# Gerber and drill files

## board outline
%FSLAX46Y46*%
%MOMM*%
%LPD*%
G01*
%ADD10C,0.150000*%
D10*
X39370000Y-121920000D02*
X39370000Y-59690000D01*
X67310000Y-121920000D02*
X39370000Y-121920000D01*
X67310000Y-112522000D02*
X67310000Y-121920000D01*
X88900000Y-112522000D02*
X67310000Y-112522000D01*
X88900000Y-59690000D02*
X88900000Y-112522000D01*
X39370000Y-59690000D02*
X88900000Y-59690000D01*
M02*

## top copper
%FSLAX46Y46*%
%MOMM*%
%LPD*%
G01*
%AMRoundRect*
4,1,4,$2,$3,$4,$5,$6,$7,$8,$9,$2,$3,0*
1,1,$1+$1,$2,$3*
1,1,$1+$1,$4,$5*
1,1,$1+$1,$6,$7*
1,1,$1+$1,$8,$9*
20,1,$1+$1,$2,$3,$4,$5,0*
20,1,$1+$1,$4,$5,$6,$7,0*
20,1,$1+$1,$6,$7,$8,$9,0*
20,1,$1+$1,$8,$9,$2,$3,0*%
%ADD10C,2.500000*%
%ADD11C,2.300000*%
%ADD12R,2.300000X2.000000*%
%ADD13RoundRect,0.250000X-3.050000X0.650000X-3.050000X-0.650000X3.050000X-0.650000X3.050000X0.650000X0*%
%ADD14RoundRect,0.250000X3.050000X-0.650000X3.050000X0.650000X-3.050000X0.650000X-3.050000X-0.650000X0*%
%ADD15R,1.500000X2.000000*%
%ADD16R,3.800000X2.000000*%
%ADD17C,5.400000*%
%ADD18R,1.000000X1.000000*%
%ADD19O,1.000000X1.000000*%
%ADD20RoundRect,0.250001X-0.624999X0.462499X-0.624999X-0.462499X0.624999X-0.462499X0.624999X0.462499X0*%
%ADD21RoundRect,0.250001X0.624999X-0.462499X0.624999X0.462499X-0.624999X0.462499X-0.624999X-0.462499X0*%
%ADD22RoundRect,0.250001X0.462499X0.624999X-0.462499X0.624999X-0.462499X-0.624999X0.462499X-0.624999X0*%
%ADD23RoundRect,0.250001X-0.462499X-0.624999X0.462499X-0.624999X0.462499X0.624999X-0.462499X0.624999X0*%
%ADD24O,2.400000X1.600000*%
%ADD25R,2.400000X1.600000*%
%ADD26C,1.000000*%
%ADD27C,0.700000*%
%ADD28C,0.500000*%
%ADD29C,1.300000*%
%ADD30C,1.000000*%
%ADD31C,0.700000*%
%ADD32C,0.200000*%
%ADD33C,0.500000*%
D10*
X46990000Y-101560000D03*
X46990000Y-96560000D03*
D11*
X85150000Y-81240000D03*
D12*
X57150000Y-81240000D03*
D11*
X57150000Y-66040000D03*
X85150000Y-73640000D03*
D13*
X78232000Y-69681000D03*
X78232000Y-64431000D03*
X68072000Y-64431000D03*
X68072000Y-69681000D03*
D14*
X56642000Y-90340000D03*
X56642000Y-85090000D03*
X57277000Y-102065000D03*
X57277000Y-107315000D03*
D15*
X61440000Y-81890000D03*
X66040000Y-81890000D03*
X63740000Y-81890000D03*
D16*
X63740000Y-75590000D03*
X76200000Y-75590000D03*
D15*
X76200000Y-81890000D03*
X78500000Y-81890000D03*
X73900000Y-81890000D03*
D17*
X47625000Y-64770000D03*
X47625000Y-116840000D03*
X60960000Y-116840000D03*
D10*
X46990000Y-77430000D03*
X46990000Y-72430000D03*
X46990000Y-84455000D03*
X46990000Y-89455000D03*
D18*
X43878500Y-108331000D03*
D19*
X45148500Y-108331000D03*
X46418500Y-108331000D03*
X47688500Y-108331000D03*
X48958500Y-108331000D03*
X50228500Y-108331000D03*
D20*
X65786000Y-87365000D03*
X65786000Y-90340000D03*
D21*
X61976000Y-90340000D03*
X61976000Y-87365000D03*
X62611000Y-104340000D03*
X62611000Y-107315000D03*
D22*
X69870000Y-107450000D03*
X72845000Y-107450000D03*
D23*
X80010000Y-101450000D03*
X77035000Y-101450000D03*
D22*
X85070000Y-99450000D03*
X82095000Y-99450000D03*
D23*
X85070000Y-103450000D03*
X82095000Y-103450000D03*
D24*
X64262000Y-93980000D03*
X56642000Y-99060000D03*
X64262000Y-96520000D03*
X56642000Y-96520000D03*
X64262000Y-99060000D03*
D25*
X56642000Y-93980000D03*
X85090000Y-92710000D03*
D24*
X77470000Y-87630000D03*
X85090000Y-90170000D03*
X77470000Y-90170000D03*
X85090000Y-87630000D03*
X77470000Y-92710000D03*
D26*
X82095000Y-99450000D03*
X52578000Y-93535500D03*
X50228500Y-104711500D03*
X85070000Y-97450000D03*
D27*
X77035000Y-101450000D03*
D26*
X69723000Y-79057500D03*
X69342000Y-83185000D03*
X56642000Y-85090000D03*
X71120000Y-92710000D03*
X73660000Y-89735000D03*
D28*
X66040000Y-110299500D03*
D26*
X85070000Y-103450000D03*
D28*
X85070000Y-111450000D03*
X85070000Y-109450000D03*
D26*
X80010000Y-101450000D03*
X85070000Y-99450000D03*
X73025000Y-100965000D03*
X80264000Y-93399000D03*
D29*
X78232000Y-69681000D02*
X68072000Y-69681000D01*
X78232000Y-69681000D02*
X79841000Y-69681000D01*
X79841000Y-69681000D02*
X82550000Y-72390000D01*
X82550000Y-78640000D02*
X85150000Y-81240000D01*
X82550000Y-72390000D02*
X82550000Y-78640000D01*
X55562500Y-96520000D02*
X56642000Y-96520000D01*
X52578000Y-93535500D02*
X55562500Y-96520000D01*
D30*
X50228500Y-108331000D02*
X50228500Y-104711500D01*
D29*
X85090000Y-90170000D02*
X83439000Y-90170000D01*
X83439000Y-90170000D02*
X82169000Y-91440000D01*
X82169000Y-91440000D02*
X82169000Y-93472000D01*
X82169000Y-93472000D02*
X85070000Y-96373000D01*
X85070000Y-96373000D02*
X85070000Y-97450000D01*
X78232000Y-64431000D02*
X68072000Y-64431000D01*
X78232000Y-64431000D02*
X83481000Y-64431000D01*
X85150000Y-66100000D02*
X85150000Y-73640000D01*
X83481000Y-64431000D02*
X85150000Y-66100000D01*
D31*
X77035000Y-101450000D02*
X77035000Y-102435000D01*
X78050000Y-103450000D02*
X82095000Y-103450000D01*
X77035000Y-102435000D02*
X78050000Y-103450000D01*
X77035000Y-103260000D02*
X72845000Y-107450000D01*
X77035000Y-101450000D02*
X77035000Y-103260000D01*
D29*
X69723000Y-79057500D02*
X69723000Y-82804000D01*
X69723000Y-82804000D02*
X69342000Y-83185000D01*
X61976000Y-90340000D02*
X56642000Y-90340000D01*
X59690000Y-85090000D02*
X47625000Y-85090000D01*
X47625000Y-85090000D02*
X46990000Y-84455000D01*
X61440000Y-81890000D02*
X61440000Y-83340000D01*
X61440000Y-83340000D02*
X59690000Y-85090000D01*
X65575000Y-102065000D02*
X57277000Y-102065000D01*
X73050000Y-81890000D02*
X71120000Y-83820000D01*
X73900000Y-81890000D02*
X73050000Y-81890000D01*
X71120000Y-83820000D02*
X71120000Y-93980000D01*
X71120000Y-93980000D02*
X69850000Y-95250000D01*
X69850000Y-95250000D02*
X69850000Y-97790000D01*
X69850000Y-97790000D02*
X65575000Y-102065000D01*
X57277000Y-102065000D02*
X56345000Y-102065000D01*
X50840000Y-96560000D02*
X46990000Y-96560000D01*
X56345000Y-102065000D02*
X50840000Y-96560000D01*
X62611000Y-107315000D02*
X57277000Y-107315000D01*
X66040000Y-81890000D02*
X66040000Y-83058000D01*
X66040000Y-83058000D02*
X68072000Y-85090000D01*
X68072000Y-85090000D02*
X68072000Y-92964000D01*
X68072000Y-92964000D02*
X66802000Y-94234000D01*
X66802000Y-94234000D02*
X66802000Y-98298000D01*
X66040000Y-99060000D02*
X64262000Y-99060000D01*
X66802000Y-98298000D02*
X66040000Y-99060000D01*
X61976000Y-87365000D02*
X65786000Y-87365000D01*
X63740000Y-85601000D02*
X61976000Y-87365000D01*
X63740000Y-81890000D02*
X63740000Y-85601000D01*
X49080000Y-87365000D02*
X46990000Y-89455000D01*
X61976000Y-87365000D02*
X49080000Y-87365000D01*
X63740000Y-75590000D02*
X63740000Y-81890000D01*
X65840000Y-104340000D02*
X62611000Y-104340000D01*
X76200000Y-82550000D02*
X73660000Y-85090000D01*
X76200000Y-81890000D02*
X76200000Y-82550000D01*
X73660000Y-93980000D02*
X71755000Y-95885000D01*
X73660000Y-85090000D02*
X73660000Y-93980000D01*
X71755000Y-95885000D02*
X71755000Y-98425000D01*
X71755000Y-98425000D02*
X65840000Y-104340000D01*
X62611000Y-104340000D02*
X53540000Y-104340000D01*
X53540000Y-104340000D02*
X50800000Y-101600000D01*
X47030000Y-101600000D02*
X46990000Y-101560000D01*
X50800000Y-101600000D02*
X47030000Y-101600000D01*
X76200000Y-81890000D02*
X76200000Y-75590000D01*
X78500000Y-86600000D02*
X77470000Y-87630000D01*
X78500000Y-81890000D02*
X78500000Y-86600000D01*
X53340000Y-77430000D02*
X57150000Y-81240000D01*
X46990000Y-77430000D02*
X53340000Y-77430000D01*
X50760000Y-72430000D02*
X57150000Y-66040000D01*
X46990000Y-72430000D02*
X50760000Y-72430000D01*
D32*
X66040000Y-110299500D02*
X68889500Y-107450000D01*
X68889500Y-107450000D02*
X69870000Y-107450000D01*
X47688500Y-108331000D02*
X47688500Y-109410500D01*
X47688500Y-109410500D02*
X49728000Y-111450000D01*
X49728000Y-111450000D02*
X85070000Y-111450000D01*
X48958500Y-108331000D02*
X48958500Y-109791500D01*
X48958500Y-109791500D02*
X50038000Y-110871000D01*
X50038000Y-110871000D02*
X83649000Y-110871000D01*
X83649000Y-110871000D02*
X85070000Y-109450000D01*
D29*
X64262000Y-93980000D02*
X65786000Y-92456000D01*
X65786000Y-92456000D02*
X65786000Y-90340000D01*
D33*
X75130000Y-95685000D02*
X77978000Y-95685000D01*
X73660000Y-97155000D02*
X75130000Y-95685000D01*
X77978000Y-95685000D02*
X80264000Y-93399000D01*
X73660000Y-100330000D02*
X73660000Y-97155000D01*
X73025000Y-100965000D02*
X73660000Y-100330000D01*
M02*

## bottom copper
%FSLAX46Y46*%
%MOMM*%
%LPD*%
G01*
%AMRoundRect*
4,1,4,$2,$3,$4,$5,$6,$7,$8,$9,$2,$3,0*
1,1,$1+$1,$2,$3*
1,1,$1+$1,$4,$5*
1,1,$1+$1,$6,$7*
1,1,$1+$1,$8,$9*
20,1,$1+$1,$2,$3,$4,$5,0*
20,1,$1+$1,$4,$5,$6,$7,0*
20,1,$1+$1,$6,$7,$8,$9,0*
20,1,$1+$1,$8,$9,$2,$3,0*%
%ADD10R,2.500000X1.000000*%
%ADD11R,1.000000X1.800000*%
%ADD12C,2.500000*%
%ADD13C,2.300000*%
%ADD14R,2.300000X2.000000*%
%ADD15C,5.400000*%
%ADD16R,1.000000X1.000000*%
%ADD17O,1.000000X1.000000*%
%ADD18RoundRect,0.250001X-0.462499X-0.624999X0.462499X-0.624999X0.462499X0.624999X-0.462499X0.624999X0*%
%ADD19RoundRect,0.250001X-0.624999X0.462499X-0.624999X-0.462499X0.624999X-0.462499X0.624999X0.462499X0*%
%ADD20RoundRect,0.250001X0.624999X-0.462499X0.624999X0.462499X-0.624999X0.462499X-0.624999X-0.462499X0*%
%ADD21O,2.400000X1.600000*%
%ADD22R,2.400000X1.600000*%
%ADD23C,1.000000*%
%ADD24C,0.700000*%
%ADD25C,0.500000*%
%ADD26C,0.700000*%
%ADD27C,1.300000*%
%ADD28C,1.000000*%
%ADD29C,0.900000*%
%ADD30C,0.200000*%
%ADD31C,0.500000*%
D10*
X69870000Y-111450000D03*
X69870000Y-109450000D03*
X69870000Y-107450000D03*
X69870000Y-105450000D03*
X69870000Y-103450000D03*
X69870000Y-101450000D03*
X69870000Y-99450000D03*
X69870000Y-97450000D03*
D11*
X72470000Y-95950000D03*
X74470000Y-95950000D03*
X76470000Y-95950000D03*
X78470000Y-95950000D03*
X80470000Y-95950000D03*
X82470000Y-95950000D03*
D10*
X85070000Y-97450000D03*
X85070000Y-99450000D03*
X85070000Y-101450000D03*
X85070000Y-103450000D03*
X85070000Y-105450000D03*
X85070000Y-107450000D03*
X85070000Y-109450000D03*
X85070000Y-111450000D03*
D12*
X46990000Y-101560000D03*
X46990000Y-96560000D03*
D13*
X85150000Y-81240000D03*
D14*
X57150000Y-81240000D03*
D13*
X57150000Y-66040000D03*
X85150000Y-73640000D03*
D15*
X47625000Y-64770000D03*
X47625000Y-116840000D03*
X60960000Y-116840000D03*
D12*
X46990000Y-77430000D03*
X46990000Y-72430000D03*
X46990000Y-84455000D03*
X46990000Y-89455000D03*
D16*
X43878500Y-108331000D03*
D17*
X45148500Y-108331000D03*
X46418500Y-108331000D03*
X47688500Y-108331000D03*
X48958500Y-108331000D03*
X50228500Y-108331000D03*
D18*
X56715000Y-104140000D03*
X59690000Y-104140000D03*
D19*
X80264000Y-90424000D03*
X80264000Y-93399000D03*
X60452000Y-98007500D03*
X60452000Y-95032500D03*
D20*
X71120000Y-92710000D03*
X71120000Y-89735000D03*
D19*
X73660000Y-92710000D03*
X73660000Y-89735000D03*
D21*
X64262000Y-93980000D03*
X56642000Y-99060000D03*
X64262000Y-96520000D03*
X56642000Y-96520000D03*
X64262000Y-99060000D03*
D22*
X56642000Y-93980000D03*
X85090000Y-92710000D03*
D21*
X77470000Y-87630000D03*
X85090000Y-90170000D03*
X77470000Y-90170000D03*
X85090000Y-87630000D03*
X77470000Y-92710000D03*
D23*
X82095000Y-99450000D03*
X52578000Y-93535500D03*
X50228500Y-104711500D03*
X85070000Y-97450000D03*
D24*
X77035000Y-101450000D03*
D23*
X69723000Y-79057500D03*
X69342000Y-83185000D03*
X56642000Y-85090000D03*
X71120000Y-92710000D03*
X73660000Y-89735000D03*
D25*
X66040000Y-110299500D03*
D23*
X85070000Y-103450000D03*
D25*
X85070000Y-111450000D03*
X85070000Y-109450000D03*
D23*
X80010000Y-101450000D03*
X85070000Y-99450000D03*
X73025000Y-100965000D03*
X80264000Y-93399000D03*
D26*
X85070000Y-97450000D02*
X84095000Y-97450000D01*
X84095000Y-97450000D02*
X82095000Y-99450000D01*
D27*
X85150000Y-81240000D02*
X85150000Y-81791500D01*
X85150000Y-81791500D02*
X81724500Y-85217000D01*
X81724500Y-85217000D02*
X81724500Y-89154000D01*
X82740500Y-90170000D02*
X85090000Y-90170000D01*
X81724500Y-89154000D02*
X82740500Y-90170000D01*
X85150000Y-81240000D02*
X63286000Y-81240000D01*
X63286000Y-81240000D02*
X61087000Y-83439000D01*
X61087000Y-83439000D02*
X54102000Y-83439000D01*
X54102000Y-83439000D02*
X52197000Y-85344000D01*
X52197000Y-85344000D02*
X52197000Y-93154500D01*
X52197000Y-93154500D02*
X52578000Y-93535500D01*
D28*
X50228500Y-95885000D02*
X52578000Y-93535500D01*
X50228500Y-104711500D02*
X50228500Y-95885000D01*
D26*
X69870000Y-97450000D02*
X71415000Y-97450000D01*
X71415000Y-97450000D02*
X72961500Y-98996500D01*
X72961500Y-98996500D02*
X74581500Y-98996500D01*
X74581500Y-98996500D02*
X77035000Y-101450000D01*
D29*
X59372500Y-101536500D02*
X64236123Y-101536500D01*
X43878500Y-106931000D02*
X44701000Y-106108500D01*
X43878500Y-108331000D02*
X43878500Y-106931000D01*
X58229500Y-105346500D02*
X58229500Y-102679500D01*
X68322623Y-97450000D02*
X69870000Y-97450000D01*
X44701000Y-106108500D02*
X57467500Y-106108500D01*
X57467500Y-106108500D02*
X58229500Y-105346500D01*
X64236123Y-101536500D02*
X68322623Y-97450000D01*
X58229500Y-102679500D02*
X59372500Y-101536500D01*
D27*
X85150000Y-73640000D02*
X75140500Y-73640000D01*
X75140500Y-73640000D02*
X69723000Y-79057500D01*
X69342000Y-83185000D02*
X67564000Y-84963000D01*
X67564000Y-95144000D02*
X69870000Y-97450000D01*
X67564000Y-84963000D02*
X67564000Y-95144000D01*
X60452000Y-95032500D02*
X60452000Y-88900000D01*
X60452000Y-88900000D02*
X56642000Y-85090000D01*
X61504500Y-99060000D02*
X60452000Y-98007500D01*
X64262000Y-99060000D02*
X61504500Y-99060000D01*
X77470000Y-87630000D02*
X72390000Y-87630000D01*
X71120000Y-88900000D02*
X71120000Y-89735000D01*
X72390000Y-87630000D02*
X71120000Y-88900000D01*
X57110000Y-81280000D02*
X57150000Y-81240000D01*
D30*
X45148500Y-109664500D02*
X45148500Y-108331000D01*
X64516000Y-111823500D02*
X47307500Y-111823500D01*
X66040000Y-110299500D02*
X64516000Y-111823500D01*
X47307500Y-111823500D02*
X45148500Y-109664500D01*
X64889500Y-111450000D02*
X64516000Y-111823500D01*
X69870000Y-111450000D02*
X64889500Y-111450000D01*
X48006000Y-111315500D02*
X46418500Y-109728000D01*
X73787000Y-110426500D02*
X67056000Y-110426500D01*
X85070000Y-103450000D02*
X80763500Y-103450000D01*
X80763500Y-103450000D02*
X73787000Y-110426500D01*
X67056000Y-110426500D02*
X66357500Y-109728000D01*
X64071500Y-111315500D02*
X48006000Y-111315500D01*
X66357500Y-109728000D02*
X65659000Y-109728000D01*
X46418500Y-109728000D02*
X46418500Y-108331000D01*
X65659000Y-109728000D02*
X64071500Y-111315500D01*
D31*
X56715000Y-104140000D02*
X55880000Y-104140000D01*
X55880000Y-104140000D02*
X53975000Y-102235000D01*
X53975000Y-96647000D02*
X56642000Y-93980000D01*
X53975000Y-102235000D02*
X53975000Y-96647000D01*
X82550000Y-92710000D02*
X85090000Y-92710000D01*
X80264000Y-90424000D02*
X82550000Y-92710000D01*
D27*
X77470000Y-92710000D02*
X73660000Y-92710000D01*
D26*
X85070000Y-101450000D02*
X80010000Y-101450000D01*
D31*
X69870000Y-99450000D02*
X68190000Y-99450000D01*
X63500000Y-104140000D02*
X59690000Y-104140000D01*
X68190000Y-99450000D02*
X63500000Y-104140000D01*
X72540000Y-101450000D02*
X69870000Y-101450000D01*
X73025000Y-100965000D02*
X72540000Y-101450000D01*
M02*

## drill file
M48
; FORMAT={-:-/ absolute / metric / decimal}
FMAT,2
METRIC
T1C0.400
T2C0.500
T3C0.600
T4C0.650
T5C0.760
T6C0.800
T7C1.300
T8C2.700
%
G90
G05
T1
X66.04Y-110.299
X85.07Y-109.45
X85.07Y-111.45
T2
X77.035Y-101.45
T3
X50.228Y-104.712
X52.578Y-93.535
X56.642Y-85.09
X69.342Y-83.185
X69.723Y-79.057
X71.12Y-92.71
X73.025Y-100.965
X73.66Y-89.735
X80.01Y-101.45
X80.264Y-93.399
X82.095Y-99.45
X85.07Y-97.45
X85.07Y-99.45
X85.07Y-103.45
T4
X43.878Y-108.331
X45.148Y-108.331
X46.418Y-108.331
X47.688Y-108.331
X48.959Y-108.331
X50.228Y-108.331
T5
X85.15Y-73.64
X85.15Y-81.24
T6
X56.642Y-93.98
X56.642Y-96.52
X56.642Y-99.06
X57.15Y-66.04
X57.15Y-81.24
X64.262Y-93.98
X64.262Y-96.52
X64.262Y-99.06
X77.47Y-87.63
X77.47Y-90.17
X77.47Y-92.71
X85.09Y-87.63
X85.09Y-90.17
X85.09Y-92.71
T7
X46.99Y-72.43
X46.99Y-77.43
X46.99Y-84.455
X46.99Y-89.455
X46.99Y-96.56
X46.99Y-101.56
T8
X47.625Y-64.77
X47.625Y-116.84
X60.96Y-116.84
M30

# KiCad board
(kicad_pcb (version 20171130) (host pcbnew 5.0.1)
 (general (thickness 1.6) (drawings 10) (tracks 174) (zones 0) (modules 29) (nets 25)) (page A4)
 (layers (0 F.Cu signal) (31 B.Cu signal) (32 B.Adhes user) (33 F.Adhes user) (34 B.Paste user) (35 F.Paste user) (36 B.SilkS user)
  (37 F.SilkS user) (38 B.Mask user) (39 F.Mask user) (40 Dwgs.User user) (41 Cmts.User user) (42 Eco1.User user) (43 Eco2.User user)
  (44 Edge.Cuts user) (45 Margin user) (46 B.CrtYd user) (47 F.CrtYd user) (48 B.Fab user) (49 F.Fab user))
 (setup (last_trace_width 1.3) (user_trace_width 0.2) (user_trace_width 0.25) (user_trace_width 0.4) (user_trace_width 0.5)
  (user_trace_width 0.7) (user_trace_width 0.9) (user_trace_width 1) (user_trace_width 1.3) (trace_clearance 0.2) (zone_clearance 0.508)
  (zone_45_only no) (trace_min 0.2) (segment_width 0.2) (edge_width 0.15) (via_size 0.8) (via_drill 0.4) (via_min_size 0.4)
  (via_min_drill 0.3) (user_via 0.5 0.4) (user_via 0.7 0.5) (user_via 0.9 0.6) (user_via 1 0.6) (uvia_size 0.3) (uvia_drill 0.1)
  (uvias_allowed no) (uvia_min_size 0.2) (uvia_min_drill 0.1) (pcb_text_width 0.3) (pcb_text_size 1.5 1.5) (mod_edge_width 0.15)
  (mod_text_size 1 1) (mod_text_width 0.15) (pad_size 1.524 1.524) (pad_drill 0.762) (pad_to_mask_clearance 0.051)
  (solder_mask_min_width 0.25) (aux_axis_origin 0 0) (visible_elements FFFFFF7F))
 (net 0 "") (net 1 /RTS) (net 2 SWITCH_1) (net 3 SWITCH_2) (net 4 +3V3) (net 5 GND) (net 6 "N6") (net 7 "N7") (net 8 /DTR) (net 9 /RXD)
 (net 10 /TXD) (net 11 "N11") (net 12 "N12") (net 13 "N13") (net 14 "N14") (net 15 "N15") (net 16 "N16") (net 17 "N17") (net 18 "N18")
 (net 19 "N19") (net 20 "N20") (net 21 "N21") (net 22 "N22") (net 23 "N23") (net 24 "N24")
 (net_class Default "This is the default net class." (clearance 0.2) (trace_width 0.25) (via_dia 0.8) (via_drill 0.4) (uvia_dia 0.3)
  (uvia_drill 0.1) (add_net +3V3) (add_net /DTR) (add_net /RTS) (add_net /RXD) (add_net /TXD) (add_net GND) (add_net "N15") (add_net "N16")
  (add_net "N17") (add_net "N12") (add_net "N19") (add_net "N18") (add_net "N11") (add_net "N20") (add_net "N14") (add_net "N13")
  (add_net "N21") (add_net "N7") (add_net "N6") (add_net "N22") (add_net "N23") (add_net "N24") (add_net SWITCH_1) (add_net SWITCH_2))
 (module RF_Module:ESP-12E (layer B.Cu) (at 77.47 107.95)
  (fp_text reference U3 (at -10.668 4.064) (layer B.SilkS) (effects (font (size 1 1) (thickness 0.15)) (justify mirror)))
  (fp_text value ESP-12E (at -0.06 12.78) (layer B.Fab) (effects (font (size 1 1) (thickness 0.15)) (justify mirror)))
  (pad 1 smd rect (at -7.6 3.5) (size 2.5 1) (layers B.Cu B.Paste B.Mask) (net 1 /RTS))
  (pad 2 smd rect (at -7.6 1.5) (size 2.5 1) (layers B.Cu B.Paste B.Mask))
  (pad 3 smd rect (at -7.6 -0.5) (size 2.5 1) (layers B.Cu B.Paste B.Mask) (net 1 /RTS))
  (pad 4 smd rect (at -7.6 -2.5) (size 2.5 1) (layers B.Cu B.Paste B.Mask))
  (pad 5 smd rect (at -7.6 -4.5) (size 2.5 1) (layers B.Cu B.Paste B.Mask))
  (pad 6 smd rect (at -7.6 -6.5) (size 2.5 1) (layers B.Cu B.Paste B.Mask) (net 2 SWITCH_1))
  (pad 7 smd rect (at -7.6 -8.5) (size 2.5 1) (layers B.Cu B.Paste B.Mask) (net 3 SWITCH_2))
  (pad 8 smd rect (at -7.6 -10.5) (size 2.5 1) (layers B.Cu B.Paste B.Mask) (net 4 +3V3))
  (pad 9 smd rect (at -5 -12) (size 1 1.8) (layers B.Cu B.Paste B.Mask))
  (pad 10 smd rect (at -3 -12) (size 1 1.8) (layers B.Cu B.Paste B.Mask))
  (pad 11 smd rect (at -1 -12) (size 1 1.8) (layers B.Cu B.Paste B.Mask))
  (pad 12 smd rect (at 1 -12) (size 1 1.8) (layers B.Cu B.Paste B.Mask))
  (pad 13 smd rect (at 3 -12) (size 1 1.8) (layers B.Cu B.Paste B.Mask))
  (pad 14 smd rect (at 5 -12) (size 1 1.8) (layers B.Cu B.Paste B.Mask))
  (pad 15 smd rect (at 7.6 -10.5) (size 2.5 1) (layers B.Cu B.Paste B.Mask) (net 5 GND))
  (pad 16 smd rect (at 7.6 -8.5) (size 2.5 1) (layers B.Cu B.Paste B.Mask) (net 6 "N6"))
  (pad 17 smd rect (at 7.6 -6.5) (size 2.5 1) (layers B.Cu B.Paste B.Mask) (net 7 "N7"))
  (pad 18 smd rect (at 7.6 -4.5) (size 2.5 1) (layers B.Cu B.Paste B.Mask) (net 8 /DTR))
  (pad 19 smd rect (at 7.6 -2.5) (size 2.5 1) (layers B.Cu B.Paste B.Mask))
  (pad 20 smd rect (at 7.6 -0.5) (size 2.5 1) (layers B.Cu B.Paste B.Mask))
  (pad 21 smd rect (at 7.6 1.5) (size 2.5 1) (layers B.Cu B.Paste B.Mask) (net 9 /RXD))
  (pad 22 smd rect (at 7.6 3.5) (size 2.5 1) (layers B.Cu B.Paste B.Mask) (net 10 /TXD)))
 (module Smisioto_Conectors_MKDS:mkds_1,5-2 (layer F.Cu) (at 46.99 99.06 270)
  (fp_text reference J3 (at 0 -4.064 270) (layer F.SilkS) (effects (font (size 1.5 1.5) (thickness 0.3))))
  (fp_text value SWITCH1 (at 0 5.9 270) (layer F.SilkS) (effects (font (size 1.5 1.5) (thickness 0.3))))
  (pad 2 thru_hole circle (at 2.5 0 270) (size 2.5 2.5) (drill 1.3) (layers *.Cu *.Mask F.SilkS) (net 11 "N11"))
  (pad 1 thru_hole circle (at -2.5 0 270) (size 2.5 2.5) (drill 1.3) (layers *.Cu *.Mask F.SilkS) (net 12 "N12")))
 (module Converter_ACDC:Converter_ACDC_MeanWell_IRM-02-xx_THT (layer B.Cu) (at 57.15 81.24)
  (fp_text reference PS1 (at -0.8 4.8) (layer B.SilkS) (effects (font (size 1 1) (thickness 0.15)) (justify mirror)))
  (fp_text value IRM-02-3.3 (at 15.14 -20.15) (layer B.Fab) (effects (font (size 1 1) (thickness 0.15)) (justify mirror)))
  (pad 3 thru_hole circle (at 28 0) (size 2.3 2.3) (drill 0.76) (layers *.Cu *.Mask) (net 5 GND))
  (pad 1 thru_hole rect (at 0 0) (size 2.3 2) (drill 0.8) (layers *.Cu *.Mask) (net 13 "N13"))
  (pad 2 thru_hole circle (at 0 -15.2) (size 2.3 2.3) (drill 0.8) (layers *.Cu *.Mask) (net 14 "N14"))
  (pad 4 thru_hole circle (at 28 -7.6) (size 2.3 2.3) (drill 0.76) (layers *.Cu *.Mask) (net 4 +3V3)))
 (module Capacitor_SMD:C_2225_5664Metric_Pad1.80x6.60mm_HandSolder (layer F.Cu) (at 78.232 67.056 270)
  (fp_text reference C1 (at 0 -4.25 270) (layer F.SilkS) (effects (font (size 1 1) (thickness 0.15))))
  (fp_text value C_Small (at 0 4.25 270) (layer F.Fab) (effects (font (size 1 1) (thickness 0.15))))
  (pad 2 smd roundrect (at 2.625 0 270) (size 1.8 6.6) (layers F.Cu F.Paste F.Mask) (roundrect_rratio 0.138889) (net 5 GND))
  (pad 1 smd roundrect (at -2.625 0 270) (size 1.8 6.6) (layers F.Cu F.Paste F.Mask) (roundrect_rratio 0.138889) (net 4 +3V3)))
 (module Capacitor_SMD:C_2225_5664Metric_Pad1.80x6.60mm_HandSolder (layer F.Cu) (at 68.072 67.056 270)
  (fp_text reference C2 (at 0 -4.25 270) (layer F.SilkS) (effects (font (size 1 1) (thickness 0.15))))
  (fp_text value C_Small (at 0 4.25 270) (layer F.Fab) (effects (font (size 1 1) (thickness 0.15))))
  (pad 1 smd roundrect (at -2.625 0 270) (size 1.8 6.6) (layers F.Cu F.Paste F.Mask) (roundrect_rratio 0.138889) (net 4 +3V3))
  (pad 2 smd roundrect (at 2.625 0 270) (size 1.8 6.6) (layers F.Cu F.Paste F.Mask) (roundrect_rratio 0.138889) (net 5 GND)))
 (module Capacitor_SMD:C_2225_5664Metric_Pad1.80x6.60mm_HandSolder (layer F.Cu) (at 56.642 87.715 90)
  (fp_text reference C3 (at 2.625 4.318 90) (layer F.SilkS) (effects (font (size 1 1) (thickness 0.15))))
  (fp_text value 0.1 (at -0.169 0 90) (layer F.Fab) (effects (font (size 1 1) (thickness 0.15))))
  (pad 1 smd roundrect (at -2.625 0 90) (size 1.8 6.6) (layers F.Cu F.Paste F.Mask) (roundrect_rratio 0.138889) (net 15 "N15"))
  (pad 2 smd roundrect (at 2.625 0 90) (size 1.8 6.6) (layers F.Cu F.Paste F.Mask) (roundrect_rratio 0.138889) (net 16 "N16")))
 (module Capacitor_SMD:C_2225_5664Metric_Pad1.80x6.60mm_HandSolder (layer F.Cu) (at 57.277 104.69 90)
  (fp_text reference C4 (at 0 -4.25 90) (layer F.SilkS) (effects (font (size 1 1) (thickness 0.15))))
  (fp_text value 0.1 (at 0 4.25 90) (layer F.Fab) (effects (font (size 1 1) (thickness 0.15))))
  (pad 2 smd roundrect (at 2.625 0 90) (size 1.8 6.6) (layers F.Cu F.Paste F.Mask) (roundrect_rratio 0.138889) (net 12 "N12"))
  (pad 1 smd roundrect (at -2.625 0 90) (size 1.8 6.6) (layers F.Cu F.Paste F.Mask) (roundrect_rratio 0.138889) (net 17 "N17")))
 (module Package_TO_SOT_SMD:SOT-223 (layer F.Cu) (at 63.74 78.74 90)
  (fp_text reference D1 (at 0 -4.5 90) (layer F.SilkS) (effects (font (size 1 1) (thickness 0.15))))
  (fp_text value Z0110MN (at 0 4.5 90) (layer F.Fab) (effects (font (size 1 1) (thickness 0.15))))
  (pad 1 smd rect (at -3.15 -2.3 90) (size 2 1.5) (layers F.Cu F.Paste F.Mask) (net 16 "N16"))
  (pad 3 smd rect (at -3.15 2.3 90) (size 2 1.5) (layers F.Cu F.Paste F.Mask) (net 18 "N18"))
  (pad 2 smd rect (at -3.15 0 90) (size 2 1.5) (layers F.Cu F.Paste F.Mask) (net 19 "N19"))
  (pad 4 smd rect (at 3.15 0 90) (size 2 3.8) (layers F.Cu F.Paste F.Mask) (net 19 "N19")))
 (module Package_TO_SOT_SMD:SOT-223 (layer F.Cu) (at 76.2 78.74 90)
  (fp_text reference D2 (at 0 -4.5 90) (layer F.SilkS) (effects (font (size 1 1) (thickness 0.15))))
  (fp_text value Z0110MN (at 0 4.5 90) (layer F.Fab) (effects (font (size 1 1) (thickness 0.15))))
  (pad 4 smd rect (at 3.15 0 90) (size 2 3.8) (layers F.Cu F.Paste F.Mask) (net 11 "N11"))
  (pad 2 smd rect (at -3.15 0 90) (size 2 1.5) (layers F.Cu F.Paste F.Mask) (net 11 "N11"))
  (pad 3 smd rect (at -3.15 2.3 90) (size 2 1.5) (layers F.Cu F.Paste F.Mask) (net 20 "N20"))
  (pad 1 smd rect (at -3.15 -2.3 90) (size 2 1.5) (layers F.Cu F.Paste F.Mask) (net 12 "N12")))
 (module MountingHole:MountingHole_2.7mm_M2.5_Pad (layer F.Cu) (at 47.625 64.77)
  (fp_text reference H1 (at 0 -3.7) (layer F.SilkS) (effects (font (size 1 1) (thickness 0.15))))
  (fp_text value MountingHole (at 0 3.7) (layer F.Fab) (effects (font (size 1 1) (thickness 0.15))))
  (pad 1 thru_hole circle (at 0 0) (size 5.4 5.4) (drill 2.7) (layers *.Cu *.Mask)))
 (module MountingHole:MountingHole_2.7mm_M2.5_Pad (layer F.Cu) (at 47.625 116.84)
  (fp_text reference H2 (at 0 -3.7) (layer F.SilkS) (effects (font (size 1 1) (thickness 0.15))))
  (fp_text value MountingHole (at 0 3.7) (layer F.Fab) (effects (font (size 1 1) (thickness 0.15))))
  (pad 1 thru_hole circle (at 0 0) (size 5.4 5.4) (drill 2.7) (layers *.Cu *.Mask)))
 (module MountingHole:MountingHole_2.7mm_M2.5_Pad (layer F.Cu) (at 60.96 116.84)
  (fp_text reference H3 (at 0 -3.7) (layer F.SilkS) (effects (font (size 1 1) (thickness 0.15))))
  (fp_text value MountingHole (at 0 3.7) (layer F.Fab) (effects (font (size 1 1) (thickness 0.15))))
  (pad 1 thru_hole circle (at 0 0) (size 5.4 5.4) (drill 2.7) (layers *.Cu *.Mask)))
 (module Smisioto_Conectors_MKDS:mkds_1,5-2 (layer F.Cu) (at 46.99 74.93 270)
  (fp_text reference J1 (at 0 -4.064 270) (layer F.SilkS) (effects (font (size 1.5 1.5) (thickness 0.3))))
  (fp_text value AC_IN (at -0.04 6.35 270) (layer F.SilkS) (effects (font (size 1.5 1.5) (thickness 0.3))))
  (pad 2 thru_hole circle (at 2.5 0 270) (size 2.5 2.5) (drill 1.3) (layers *.Cu *.Mask F.SilkS) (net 13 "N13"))
  (pad 1 thru_hole circle (at -2.5 0 270) (size 2.5 2.5) (drill 1.3) (layers *.Cu *.Mask F.SilkS) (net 14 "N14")))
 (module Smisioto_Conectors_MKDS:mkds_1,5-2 (layer F.Cu) (at 46.99 86.955 270)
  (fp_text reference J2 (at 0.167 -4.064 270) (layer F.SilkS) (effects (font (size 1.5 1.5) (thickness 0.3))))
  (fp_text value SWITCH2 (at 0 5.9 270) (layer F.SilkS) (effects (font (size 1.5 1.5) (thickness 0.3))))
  (pad 1 thru_hole circle (at -2.5 0 270) (size 2.5 2.5) (drill 1.3) (layers *.Cu *.Mask F.SilkS) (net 16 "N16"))
  (pad 2 thru_hole circle (at 2.5 0 270) (size 2.5 2.5) (drill 1.3) (layers *.Cu *.Mask F.SilkS) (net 19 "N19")))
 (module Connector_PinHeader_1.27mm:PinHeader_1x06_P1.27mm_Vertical (layer F.Cu) (at 43.8785 108.331 90)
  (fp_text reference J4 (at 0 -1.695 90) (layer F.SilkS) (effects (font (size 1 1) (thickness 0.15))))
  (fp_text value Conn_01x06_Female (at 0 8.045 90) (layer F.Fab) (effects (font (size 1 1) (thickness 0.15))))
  (pad 1 thru_hole rect (at 0 0 90) (size 1 1) (drill 0.65) (layers *.Cu *.Mask) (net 4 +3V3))
  (pad 2 thru_hole oval (at 0 1.27 90) (size 1 1) (drill 0.65) (layers *.Cu *.Mask) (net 1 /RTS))
  (pad 3 thru_hole oval (at 0 2.54 90) (size 1 1) (drill 0.65) (layers *.Cu *.Mask) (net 8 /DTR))
  (pad 4 thru_hole oval (at 0 3.81 90) (size 1 1) (drill 0.65) (layers *.Cu *.Mask) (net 10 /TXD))
  (pad 5 thru_hole oval (at 0 5.08 90) (size 1 1) (drill 0.65) (layers *.Cu *.Mask) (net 9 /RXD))
  (pad 6 thru_hole oval (at 0 6.35 90) (size 1 1) (drill 0.65) (layers *.Cu *.Mask) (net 5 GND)))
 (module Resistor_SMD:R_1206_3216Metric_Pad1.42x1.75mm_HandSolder (layer B.Cu) (at 58.2025 104.14)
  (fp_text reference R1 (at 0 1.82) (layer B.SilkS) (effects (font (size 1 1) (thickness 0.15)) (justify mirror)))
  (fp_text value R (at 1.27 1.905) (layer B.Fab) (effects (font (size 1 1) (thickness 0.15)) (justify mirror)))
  (pad 1 smd roundrect (at -1.4875 0) (size 1.425 1.75) (layers B.Cu B.Paste B.Mask) (roundrect_rratio 0.175439) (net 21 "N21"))
  (pad 2 smd roundrect (at 1.4875 0) (size 1.425 1.75) (layers B.Cu B.Paste B.Mask) (roundrect_rratio 0.175439) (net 3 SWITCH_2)))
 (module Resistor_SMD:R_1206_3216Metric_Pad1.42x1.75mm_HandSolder (layer B.Cu) (at 80.264 91.9115 270)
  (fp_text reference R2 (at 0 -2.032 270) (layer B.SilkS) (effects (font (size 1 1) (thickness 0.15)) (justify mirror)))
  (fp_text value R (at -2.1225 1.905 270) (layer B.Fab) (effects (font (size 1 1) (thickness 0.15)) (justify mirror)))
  (pad 1 smd roundrect (at -1.4875 0 270) (size 1.425 1.75) (layers B.Cu B.Paste B.Mask) (roundrect_rratio 0.175439) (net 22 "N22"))
  (pad 2 smd roundrect (at 1.4875 0 270) (size 1.425 1.75) (layers B.Cu B.Paste B.Mask) (roundrect_rratio 0.175439) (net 2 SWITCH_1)))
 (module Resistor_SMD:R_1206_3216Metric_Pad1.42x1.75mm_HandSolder (layer B.Cu) (at 60.452 96.52 270)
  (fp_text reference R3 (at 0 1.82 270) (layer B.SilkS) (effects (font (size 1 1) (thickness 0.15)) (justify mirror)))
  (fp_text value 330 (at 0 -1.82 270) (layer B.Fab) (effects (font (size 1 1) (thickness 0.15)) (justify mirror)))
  (pad 2 smd roundrect (at 1.4875 0 270) (size 1.425 1.75) (layers B.Cu B.Paste B.Mask) (roundrect_rratio 0.175439) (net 18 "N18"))
  (pad 1 smd roundrect (at -1.4875 0 270) (size 1.425 1.75) (layers B.Cu B.Paste B.Mask) (roundrect_rratio 0.175439) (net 16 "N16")))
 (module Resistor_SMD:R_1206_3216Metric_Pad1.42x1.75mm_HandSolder (layer B.Cu) (at 71.12 91.2225 90)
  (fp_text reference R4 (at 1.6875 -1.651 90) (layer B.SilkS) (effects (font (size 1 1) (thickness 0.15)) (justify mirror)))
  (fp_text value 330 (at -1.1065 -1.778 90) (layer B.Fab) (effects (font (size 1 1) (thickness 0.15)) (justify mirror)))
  (pad 1 smd roundrect (at -1.4875 0 90) (size 1.425 1.75) (layers B.Cu B.Paste B.Mask) (roundrect_rratio 0.175439) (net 12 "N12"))
  (pad 2 smd roundrect (at 1.4875 0 90) (size 1.425 1.75) (layers B.Cu B.Paste B.Mask) (roundrect_rratio 0.175439) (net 20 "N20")))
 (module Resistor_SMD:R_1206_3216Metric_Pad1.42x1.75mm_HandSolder (layer F.Cu) (at 65.786 88.8525 270)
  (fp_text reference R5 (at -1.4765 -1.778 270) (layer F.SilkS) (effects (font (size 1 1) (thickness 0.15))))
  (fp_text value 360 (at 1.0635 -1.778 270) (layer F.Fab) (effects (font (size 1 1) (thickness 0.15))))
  (pad 1 smd roundrect (at -1.4875 0 270) (size 1.425 1.75) (layers F.Cu F.Paste F.Mask) (roundrect_rratio 0.175439) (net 19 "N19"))
  (pad 2 smd roundrect (at 1.4875 0 270) (size 1.425 1.75) (layers F.Cu F.Paste F.Mask) (roundrect_rratio 0.175439) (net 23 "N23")))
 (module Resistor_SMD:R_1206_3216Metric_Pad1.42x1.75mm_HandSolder (layer B.Cu) (at 73.66 91.2225 270)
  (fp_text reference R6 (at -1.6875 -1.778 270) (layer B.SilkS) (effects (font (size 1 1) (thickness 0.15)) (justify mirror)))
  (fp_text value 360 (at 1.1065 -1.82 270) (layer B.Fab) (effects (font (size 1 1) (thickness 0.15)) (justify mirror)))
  (pad 2 smd roundrect (at 1.4875 0 270) (size 1.425 1.75) (layers B.Cu B.Paste B.Mask) (roundrect_rratio 0.175439) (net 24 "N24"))
  (pad 1 smd roundrect (at -1.4875 0 270) (size 1.425 1.75) (layers B.Cu B.Paste B.Mask) (roundrect_rratio 0.175439) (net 11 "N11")))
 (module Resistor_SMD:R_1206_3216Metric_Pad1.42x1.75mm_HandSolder (layer F.Cu) (at 61.976 88.8525 90)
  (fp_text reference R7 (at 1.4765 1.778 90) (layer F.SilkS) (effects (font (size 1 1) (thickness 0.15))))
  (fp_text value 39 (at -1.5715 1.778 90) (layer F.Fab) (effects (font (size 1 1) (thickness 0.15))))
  (pad 1 smd roundrect (at -1.4875 0 90) (size 1.425 1.75) (layers F.Cu F.Paste F.Mask) (roundrect_rratio 0.175439) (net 15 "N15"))
  (pad 2 smd roundrect (at 1.4875 0 90) (size 1.425 1.75) (layers F.Cu F.Paste F.Mask) (roundrect_rratio 0.175439) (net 19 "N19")))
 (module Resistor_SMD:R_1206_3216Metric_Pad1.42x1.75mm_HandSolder (layer F.Cu) (at 62.611 105.8275 90)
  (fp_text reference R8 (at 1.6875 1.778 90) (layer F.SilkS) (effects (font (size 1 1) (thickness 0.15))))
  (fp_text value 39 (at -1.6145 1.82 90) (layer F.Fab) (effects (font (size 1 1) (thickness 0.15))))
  (pad 2 smd roundrect (at 1.4875 0 90) (size 1.425 1.75) (layers F.Cu F.Paste F.Mask) (roundrect_rratio 0.175439) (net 11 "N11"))
  (pad 1 smd roundrect (at -1.4875 0 90) (size 1.425 1.75) (layers F.Cu F.Paste F.Mask) (roundrect_rratio 0.175439) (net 17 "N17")))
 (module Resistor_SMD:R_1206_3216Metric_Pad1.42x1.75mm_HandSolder (layer F.Cu) (at 71.3575 107.45 180)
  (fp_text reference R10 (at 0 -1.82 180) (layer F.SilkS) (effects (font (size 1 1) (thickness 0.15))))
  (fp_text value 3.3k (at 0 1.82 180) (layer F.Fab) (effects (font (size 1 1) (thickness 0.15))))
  (pad 2 smd roundrect (at 1.4875 0 180) (size 1.425 1.75) (layers F.Cu F.Paste F.Mask) (roundrect_rratio 0.175439) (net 1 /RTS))
  (pad 1 smd roundrect (at -1.4875 0 180) (size 1.425 1.75) (layers F.Cu F.Paste F.Mask) (roundrect_rratio 0.175439) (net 4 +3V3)))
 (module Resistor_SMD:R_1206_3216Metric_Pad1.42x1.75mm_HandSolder (layer F.Cu) (at 78.5225 101.45)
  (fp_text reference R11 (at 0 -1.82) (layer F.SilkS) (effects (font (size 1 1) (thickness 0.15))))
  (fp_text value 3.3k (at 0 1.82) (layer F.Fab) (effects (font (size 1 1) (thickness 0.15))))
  (pad 2 smd roundrect (at 1.4875 0) (size 1.425 1.75) (layers F.Cu F.Paste F.Mask) (roundrect_rratio 0.175439) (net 7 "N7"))
  (pad 1 smd roundrect (at -1.4875 0) (size 1.425 1.75) (layers F.Cu F.Paste F.Mask) (roundrect_rratio 0.175439) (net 4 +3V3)))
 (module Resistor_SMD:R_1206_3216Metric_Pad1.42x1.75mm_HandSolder (layer F.Cu) (at 83.5825 99.45 180)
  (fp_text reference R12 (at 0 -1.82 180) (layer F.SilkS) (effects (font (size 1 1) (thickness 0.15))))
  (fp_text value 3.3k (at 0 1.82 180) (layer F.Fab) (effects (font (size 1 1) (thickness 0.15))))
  (pad 1 smd roundrect (at -1.4875 0 180) (size 1.425 1.75) (layers F.Cu F.Paste F.Mask) (roundrect_rratio 0.175439) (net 6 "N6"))
  (pad 2 smd roundrect (at 1.4875 0 180) (size 1.425 1.75) (layers F.Cu F.Paste F.Mask) (roundrect_rratio 0.175439) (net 5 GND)))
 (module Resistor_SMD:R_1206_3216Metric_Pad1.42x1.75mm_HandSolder (layer F.Cu) (at 83.5825 103.45)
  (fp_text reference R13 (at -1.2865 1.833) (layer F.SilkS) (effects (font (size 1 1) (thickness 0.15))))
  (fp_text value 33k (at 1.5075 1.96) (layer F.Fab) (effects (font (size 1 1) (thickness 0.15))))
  (pad 2 smd roundrect (at 1.4875 0) (size 1.425 1.75) (layers F.Cu F.Paste F.Mask) (roundrect_rratio 0.175439) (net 8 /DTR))
  (pad 1 smd roundrect (at -1.4875 0) (size 1.425 1.75) (layers F.Cu F.Paste F.Mask) (roundrect_rratio 0.175439) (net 4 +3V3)))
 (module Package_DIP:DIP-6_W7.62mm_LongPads (layer F.Cu) (at 56.642 93.98)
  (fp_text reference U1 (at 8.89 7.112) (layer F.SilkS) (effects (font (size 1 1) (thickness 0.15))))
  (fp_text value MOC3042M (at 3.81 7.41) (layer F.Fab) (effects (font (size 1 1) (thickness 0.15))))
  (pad 6 thru_hole oval (at 7.62 0) (size 2.4 1.6) (drill 0.8) (layers *.Cu *.Mask) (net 23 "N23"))
  (pad 3 thru_hole oval (at 0 5.08) (size 2.4 1.6) (drill 0.8) (layers *.Cu *.Mask))
  (pad 5 thru_hole oval (at 7.62 2.54) (size 2.4 1.6) (drill 0.8) (layers *.Cu *.Mask))
  (pad 2 thru_hole oval (at 0 2.54) (size 2.4 1.6) (drill 0.8) (layers *.Cu *.Mask) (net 5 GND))
  (pad 4 thru_hole oval (at 7.62 5.08) (size 2.4 1.6) (drill 0.8) (layers *.Cu *.Mask) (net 18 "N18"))
  (pad 1 thru_hole rect (at 0 0) (size 2.4 1.6) (drill 0.8) (layers *.Cu *.Mask) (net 21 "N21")))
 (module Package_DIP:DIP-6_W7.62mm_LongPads (layer F.Cu) (at 85.09 92.71 180)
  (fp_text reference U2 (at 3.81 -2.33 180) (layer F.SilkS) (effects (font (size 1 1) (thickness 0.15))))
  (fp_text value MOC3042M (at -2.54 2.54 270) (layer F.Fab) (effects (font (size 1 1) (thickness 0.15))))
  (pad 1 thru_hole rect (at 0 0 180) (size 2.4 1.6) (drill 0.8) (layers *.Cu *.Mask) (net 22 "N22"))
  (pad 4 thru_hole oval (at 7.62 5.08 180) (size 2.4 1.6) (drill 0.8) (layers *.Cu *.Mask) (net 20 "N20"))
  (pad 2 thru_hole oval (at 0 2.54 180) (size 2.4 1.6) (drill 0.8) (layers *.Cu *.Mask) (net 5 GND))
  (pad 5 thru_hole oval (at 7.62 2.54 180) (size 2.4 1.6) (drill 0.8) (layers *.Cu *.Mask))
  (pad 3 thru_hole oval (at 0 5.08 180) (size 2.4 1.6) (drill 0.8) (layers *.Cu *.Mask))
  (pad 6 thru_hole oval (at 7.62 0 180) (size 2.4 1.6) (drill 0.8) (layers *.Cu *.Mask) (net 24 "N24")))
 (gr_line (start 39.37 121.92) (end 39.37 59.69) (layer Edge.Cuts) (width 0.15))
 (gr_line (start 67.31 121.92) (end 39.37 121.92) (layer Edge.Cuts) (width 0.15))
 (gr_line (start 67.31 112.522) (end 67.31 121.92) (layer Edge.Cuts) (width 0.15))
 (gr_line (start 88.9 112.522) (end 67.31 112.522) (layer Edge.Cuts) (width 0.15))
 (gr_line (start 88.9 59.69) (end 88.9 112.522) (layer Edge.Cuts) (width 0.15))
 (gr_line (start 39.37 59.69) (end 88.9 59.69) (layer Edge.Cuts) (width 0.15))
 (segment (start 78.232 69.681) (end 68.072 69.681) (width 1.3) (layer F.Cu) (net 5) (status 30))
 (segment (start 78.232 69.681) (end 79.841 69.681) (width 1.3) (layer F.Cu) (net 5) (status 30))
 (segment (start 79.841 69.681) (end 82.55 72.39) (width 1.3) (layer F.Cu) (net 5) (status 10))
 (segment (start 82.55 78.64) (end 85.15 81.24) (width 1.3) (layer F.Cu) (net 5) (status 20))
 (segment (start 82.55 72.39) (end 82.55 78.64) (width 1.3) (layer F.Cu) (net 5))
 (segment (start 85.07 97.45) (end 84.095 97.45) (width 0.7) (layer B.Cu) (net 5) (status 30))
 (via (at 82.095 99.45) (size 1) (drill 0.6) (layers F.Cu B.Cu) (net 5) (status 30))
 (segment (start 84.095 97.45) (end 82.095 99.45) (width 0.7) (layer B.Cu) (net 5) (status 10))
 (segment (start 85.15 81.24) (end 85.15 81.7915) (width 1.3) (layer B.Cu) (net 5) (status 30))
 (segment (start 85.15 81.7915) (end 81.7245 85.217) (width 1.3) (layer B.Cu) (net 5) (status 10))
 (segment (start 81.7245 85.217) (end 81.7245 89.154) (width 1.3) (layer B.Cu) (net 5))
 (segment (start 82.7405 90.17) (end 85.09 90.17) (width 1.3) (layer B.Cu) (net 5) (status 20))
 (segment (start 81.7245 89.154) (end 82.7405 90.17) (width 1.3) (layer B.Cu) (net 5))
 (segment (start 85.15 81.24) (end 63.286 81.24) (width 1.3) (layer B.Cu) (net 5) (status 10))
 (segment (start 63.286 81.24) (end 61.087 83.439) (width 1.3) (layer B.Cu) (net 5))
 (segment (start 61.087 83.439) (end 54.102 83.439) (width 1.3) (layer B.Cu) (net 5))
 (segment (start 54.102 83.439) (end 52.197 85.344) (width 1.3) (layer B.Cu) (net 5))
 (via (at 52.578 93.5355) (size 1) (drill 0.6) (layers F.Cu B.Cu) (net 5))
 (segment (start 52.197 85.344) (end 52.197 93.1545) (width 1.3) (layer B.Cu) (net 5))
 (segment (start 52.197 93.1545) (end 52.578 93.5355) (width 1.3) (layer B.Cu) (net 5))
 (segment (start 55.5625 96.52) (end 56.642 96.52) (width 1.3) (layer F.Cu) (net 5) (status 30))
 (segment (start 52.578 93.5355) (end 55.5625 96.52) (width 1.3) (layer F.Cu) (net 5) (status 20))
 (via (at 50.2285 104.7115) (size 1) (drill 0.6) (layers F.Cu B.Cu) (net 5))
 (segment (start 50.2285 108.331) (end 50.2285 104.7115) (width 1) (layer F.Cu) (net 5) (status 10))
 (segment (start 50.2285 95.885) (end 52.578 93.5355) (width 1) (layer B.Cu) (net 5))
 (segment (start 50.2285 104.7115) (end 50.2285 95.885) (width 1) (layer B.Cu) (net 5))
 (segment (start 85.09 90.17) (end 83.439 90.17) (width 1.3) (layer F.Cu) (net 5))
 (segment (start 83.439 90.17) (end 82.169 91.44) (width 1.3) (layer F.Cu) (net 5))
 (segment (start 82.169 91.44) (end 82.169 93.472) (width 1.3) (layer F.Cu) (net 5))
 (via (at 85.07 97.45) (size 1) (drill 0.6) (layers F.Cu B.Cu) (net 5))
 (segment (start 82.169 93.472) (end 85.07 96.373) (width 1.3) (layer F.Cu) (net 5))
 (segment (start 85.07 96.373) (end 85.07 97.45) (width 1.3) (layer F.Cu) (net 5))
 (segment (start 78.232 64.431) (end 68.072 64.431) (width 1.3) (layer F.Cu) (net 4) (status 30))
 (segment (start 78.232 64.431) (end 83.481 64.431) (width 1.3) (layer F.Cu) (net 4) (status 10))
 (segment (start 85.15 66.1) (end 85.15 73.64) (width 1.3) (layer F.Cu) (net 4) (status 20))
 (segment (start 83.481 64.431) (end 85.15 66.1) (width 1.3) (layer F.Cu) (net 4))
 (segment (start 77.035 101.45) (end 77.035 102.435) (width 0.7) (layer F.Cu) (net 4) (status 10))
 (segment (start 78.05 103.45) (end 82.095 103.45) (width 0.7) (layer F.Cu) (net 4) (status 20))
 (segment (start 77.035 102.435) (end 78.05 103.45) (width 0.7) (layer F.Cu) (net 4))
 (segment (start 77.035 103.26) (end 72.845 107.45) (width 0.7) (layer F.Cu) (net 4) (status 20))
 (segment (start 77.035 101.45) (end 77.035 103.26) (width 0.7) (layer F.Cu) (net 4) (status 10))
 (segment (start 69.87 97.45) (end 71.415 97.45) (width 0.7) (layer B.Cu) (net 4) (status 10))
 (segment (start 71.415 97.45) (end 72.9615 98.9965) (width 0.7) (layer B.Cu) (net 4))
 (via (at 77.035 101.45) (size 0.7) (drill 0.5) (layers F.Cu B.Cu) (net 4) (status 30))
 (segment (start 72.9615 98.9965) (end 74.5815 98.9965) (width 0.7) (layer B.Cu) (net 4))
 (segment (start 74.5815 98.9965) (end 77.035 101.45) (width 0.7) (layer B.Cu) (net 4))
 (segment (start 59.3725 101.5365) (end 64.236123 101.5365) (width 0.9) (layer B.Cu) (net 4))
 (segment (start 43.8785 106.931) (end 44.701 106.1085) (width 0.9) (layer B.Cu) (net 4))
 (segment (start 43.8785 108.331) (end 43.8785 106.931) (width 0.9) (layer B.Cu) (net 4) (status 10))
 (segment (start 58.2295 105.3465) (end 58.2295 102.6795) (width 0.9) (layer B.Cu) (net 4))
 (segment (start 68.322623 97.45) (end 69.87 97.45) (width 0.9) (layer B.Cu) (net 4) (status 20))
 (segment (start 44.701 106.1085) (end 57.4675 106.1085) (width 0.9) (layer B.Cu) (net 4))
 (segment (start 57.4675 106.1085) (end 58.2295 105.3465) (width 0.9) (layer B.Cu) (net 4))
 (segment (start 64.236123 101.5365) (end 68.322623 97.45) (width 0.9) (layer B.Cu) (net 4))
 (segment (start 58.2295 102.6795) (end 59.3725 101.5365) (width 0.9) (layer B.Cu) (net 4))
 (via (at 69.723 79.0575) (size 1) (drill 0.6) (layers F.Cu B.Cu) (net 4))
 (segment (start 85.15 73.64) (end 75.1405 73.64) (width 1.3) (layer B.Cu) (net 4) (status 10))
 (segment (start 75.1405 73.64) (end 69.723 79.0575) (width 1.3) (layer B.Cu) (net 4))
 (via (at 69.342 83.185) (size 1) (drill 0.6) (layers F.Cu B.Cu) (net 4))
 (segment (start 69.723 79.0575) (end 69.723 82.804) (width 1.3) (layer F.Cu) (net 4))
 (segment (start 69.723 82.804) (end 69.342 83.185) (width 1.3) (layer F.Cu) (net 4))
 (segment (start 69.342 83.185) (end 67.564 84.963) (width 1.3) (layer B.Cu) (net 4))
 (segment (start 67.564 95.144) (end 69.87 97.45) (width 1.3) (layer B.Cu) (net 4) (status 20))
 (segment (start 67.564 84.963) (end 67.564 95.144) (width 1.3) (layer B.Cu) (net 4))
 (segment (start 61.976 90.34) (end 56.642 90.34) (width 1.3) (layer F.Cu) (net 15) (status 30))
 (via (at 56.642 85.09) (size 1) (drill 0.6) (layers F.Cu B.Cu) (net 16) (status 30))
 (segment (start 60.452 95.0325) (end 60.452 88.9) (width 1.3) (layer B.Cu) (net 16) (status 10))
 (segment (start 60.452 88.9) (end 56.642 85.09) (width 1.3) (layer B.Cu) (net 16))
 (segment (start 59.69 85.09) (end 47.625 85.09) (width 1.3) (layer F.Cu) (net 16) (status 30))
 (segment (start 47.625 85.09) (end 46.99 84.455) (width 1.3) (layer F.Cu) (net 16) (status 30))
 (segment (start 61.44 81.89) (end 61.44 83.34) (width 1.3) (layer F.Cu) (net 16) (status 10))
 (segment (start 61.44 83.34) (end 59.69 85.09) (width 1.3) (layer F.Cu) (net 16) (status 20))
 (via (at 71.12 92.71) (size 1) (drill 0.6) (layers F.Cu B.Cu) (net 12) (status 30))
 (segment (start 65.575 102.065) (end 57.277 102.065) (width 1.3) (layer F.Cu) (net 12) (status 20))
 (segment (start 73.05 81.89) (end 71.12 83.82) (width 1.3) (layer F.Cu) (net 12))
 (segment (start 73.9 81.89) (end 73.05 81.89) (width 1.3) (layer F.Cu) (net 12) (status 10))
 (segment (start 71.12 83.82) (end 71.12 93.98) (width 1.3) (layer F.Cu) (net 12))
 (segment (start 71.12 93.98) (end 69.85 95.25) (width 1.3) (layer F.Cu) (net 12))
 (segment (start 69.85 95.25) (end 69.85 97.79) (width 1.3) (layer F.Cu) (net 12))
 (segment (start 69.85 97.79) (end 65.575 102.065) (width 1.3) (layer F.Cu) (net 12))
 (segment (start 57.277 102.065) (end 56.345 102.065) (width 1.3) (layer F.Cu) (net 12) (status 30))
 (segment (start 50.84 96.56) (end 46.99 96.56) (width 1.3) (layer F.Cu) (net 12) (status 20))
 (segment (start 56.345 102.065) (end 50.84 96.56) (width 1.3) (layer F.Cu) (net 12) (status 10))
 (segment (start 62.611 107.315) (end 57.277 107.315) (width 1.3) (layer F.Cu) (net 17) (status 30))
 (segment (start 61.5045 99.06) (end 60.452 98.0075) (width 1.3) (layer B.Cu) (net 18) (status 20))
 (segment (start 64.262 99.06) (end 61.5045 99.06) (width 1.3) (layer B.Cu) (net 18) (status 10))
 (segment (start 66.04 81.89) (end 66.04 83.058) (width 1.3) (layer F.Cu) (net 18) (status 10))
 (segment (start 66.04 83.058) (end 68.072 85.09) (width 1.3) (layer F.Cu) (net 18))
 (segment (start 68.072 85.09) (end 68.072 92.964) (width 1.3) (layer F.Cu) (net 18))
 (segment (start 68.072 92.964) (end 66.802 94.234) (width 1.3) (layer F.Cu) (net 18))
 (segment (start 66.802 94.234) (end 66.802 98.298) (width 1.3) (layer F.Cu) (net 18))
 (segment (start 66.04 99.06) (end 64.262 99.06) (width 1.3) (layer F.Cu) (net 18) (status 20))
 (segment (start 66.802 98.298) (end 66.04 99.06) (width 1.3) (layer F.Cu) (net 18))
 (segment (start 61.976 87.365) (end 65.786 87.365) (width 1.3) (layer F.Cu) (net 19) (status 30))
 (segment (start 63.74 85.601) (end 61.976 87.365) (width 1.3) (layer F.Cu) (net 19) (status 20))
 (segment (start 63.74 81.89) (end 63.74 85.601) (width 1.3) (layer F.Cu) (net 19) (status 10))
 (segment (start 49.08 87.365) (end 46.99 89.455) (width 1.3) (layer F.Cu) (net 19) (status 20))
 (segment (start 61.976 87.365) (end 49.08 87.365) (width 1.3) (layer F.Cu) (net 19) (status 10))
 (segment (start 63.74 75.59) (end 63.74 81.89) (width 1.3) (layer F.Cu) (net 19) (status 30))
 (via (at 73.66 89.735) (size 1) (drill 0.6) (layers F.Cu B.Cu) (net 11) (status 30))
 (segment (start 65.84 104.34) (end 62.611 104.34) (width 1.3) (layer F.Cu) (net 11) (status 20))
 (segment (start 76.2 82.55) (end 73.66 85.09) (width 1.3) (layer F.Cu) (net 11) (status 10))
 (segment (start 76.2 81.89) (end 76.2 82.55) (width 1.3) (layer F.Cu) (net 11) (status 30))
 (segment (start 73.66 93.98) (end 71.755 95.885) (width 1.3) (layer F.Cu) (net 11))
 (segment (start 73.66 85.09) (end 73.66 93.98) (width 1.3) (layer F.Cu) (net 11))
 (segment (start 71.755 95.885) (end 71.755 98.425) (width 1.3) (layer F.Cu) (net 11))
 (segment (start 71.755 98.425) (end 65.84 104.34) (width 1.3) (layer F.Cu) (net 11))
 (segment (start 62.611 104.34) (end 53.54 104.34) (width 1.3) (layer F.Cu) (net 11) (status 10))
 (segment (start 53.54 104.34) (end 50.8 101.6) (width 1.3) (layer F.Cu) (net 11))
 (segment (start 47.03 101.6) (end 46.99 101.56) (width 1.3) (layer F.Cu) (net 11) (status 30))
 (segment (start 50.8 101.6) (end 47.03 101.6) (width 1.3) (layer F.Cu) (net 11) (status 20))
 (segment (start 76.2 81.89) (end 76.2 75.59) (width 1.3) (layer F.Cu) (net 11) (status 30))
 (segment (start 78.5 86.6) (end 77.47 87.63) (width 1.3) (layer F.Cu) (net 20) (status 20))
 (segment (start 78.5 81.89) (end 78.5 86.6) (width 1.3) (layer F.Cu) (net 20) (status 10))
 (segment (start 77.47 87.63) (end 72.39 87.63) (width 1.3) (layer B.Cu) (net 20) (status 10))
 (segment (start 71.12 88.9) (end 71.12 89.735) (width 1.3) (layer B.Cu) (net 20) (status 20))
 (segment (start 72.39 87.63) (end 71.12 88.9) (width 1.3) (layer B.Cu) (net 20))
 (segment (start 57.11 81.28) (end 57.15 81.24) (width 1.3) (layer B.Cu) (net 13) (status 30))
 (segment (start 53.34 77.43) (end 57.15 81.24) (width 1.3) (layer F.Cu) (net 13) (status 20))
 (segment (start 46.99 77.43) (end 53.34 77.43) (width 1.3) (layer F.Cu) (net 13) (status 10))
 (segment (start 50.76 72.43) (end 57.15 66.04) (width 1.3) (layer F.Cu) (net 14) (status 20))
 (segment (start 46.99 72.43) (end 50.76 72.43) (width 1.3) (layer F.Cu) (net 14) (status 10))
 (segment (start 45.1485 109.6645) (end 45.1485 108.331) (width 0.2) (layer B.Cu) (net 1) (status 20))
 (segment (start 66.04 110.2995) (end 68.8895 107.45) (width 0.2) (layer F.Cu) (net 1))
 (via (at 66.04 110.2995) (size 0.5) (drill 0.4) (layers F.Cu B.Cu) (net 1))
 (segment (start 68.8895 107.45) (end 69.87 107.45) (width 0.2) (layer F.Cu) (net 1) (status 20))
 (segment (start 64.516 111.8235) (end 47.3075 111.8235) (width 0.2) (layer B.Cu) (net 1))
 (segment (start 66.04 110.2995) (end 64.516 111.8235) (width 0.2) (layer B.Cu) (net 1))
 (segment (start 47.3075 111.8235) (end 45.1485 109.6645) (width 0.2) (layer B.Cu) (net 1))
 (segment (start 64.8895 111.45) (end 64.516 111.8235) (width 0.2) (layer B.Cu) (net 1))
 (segment (start 69.87 111.45) (end 64.8895 111.45) (width 0.2) (layer B.Cu) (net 1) (status 10))
 (via (at 85.07 103.45) (size 1) (drill 0.6) (layers F.Cu B.Cu) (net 8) (status 30))
 (segment (start 48.006 111.3155) (end 46.4185 109.728) (width 0.2) (layer B.Cu) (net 8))
 (segment (start 73.787 110.4265) (end 67.056 110.4265) (width 0.2) (layer B.Cu) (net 8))
 (segment (start 85.07 103.45) (end 80.7635 103.45) (width 0.2) (layer B.Cu) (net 8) (status 10))
 (segment (start 80.7635 103.45) (end 73.787 110.4265) (width 0.2) (layer B.Cu) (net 8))
 (segment (start 67.056 110.4265) (end 66.3575 109.728) (width 0.2) (layer B.Cu) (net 8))
 (segment (start 64.0715 111.3155) (end 48.006 111.3155) (width 0.2) (layer B.Cu) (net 8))
 (segment (start 66.3575 109.728) (end 65.659 109.728) (width 0.2) (layer B.Cu) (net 8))
 (segment (start 46.4185 109.728) (end 46.4185 108.331) (width 0.2) (layer B.Cu) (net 8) (status 20))
 (segment (start 65.659 109.728) (end 64.0715 111.3155) (width 0.2) (layer B.Cu) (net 8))
 (segment (start 47.6885 108.331) (end 47.6885 109.4105) (width 0.2) (layer F.Cu) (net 10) (status 10))
 (via (at 85.07 111.45) (size 0.5) (drill 0.4) (layers F.Cu B.Cu) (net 10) (status 30))
 (segment (start 47.6885 109.4105) (end 49.728 111.45) (width 0.2) (layer F.Cu) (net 10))
 (segment (start 49.728 111.45) (end 85.07 111.45) (width 0.2) (layer F.Cu) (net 10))
 (segment (start 48.9585 108.331) (end 48.9585 109.7915) (width 0.2) (layer F.Cu) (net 9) (status 10))
 (segment (start 48.9585 109.7915) (end 50.038 110.871) (width 0.2) (layer F.Cu) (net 9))
 (via (at 85.07 109.45) (size 0.5) (drill 0.4) (layers F.Cu B.Cu) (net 9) (status 30))
 (segment (start 50.038 110.871) (end 83.649 110.871) (width 0.2) (layer F.Cu) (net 9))
 (segment (start 83.649 110.871) (end 85.07 109.45) (width 0.2) (layer F.Cu) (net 9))
 (segment (start 56.715 104.14) (end 55.88 104.14) (width 0.5) (layer B.Cu) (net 21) (status 10))
 (segment (start 55.88 104.14) (end 53.975 102.235) (width 0.5) (layer B.Cu) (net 21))
 (segment (start 53.975 96.647) (end 56.642 93.98) (width 0.5) (layer B.Cu) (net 21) (status 20))
 (segment (start 53.975 102.235) (end 53.975 96.647) (width 0.5) (layer B.Cu) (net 21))
 (segment (start 82.55 92.71) (end 85.09 92.71) (width 0.5) (layer B.Cu) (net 22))
 (segment (start 80.264 90.424) (end 82.55 92.71) (width 0.5) (layer B.Cu) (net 22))
 (segment (start 64.262 93.98) (end 65.786 92.456) (width 1.3) (layer F.Cu) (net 23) (status 10))
 (segment (start 65.786 92.456) (end 65.786 90.34) (width 1.3) (layer F.Cu) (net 23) (status 20))
 (segment (start 77.47 92.71) (end 73.66 92.71) (width 1.3) (layer B.Cu) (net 24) (status 30))
 (via (at 80.01 101.45) (size 1) (drill 0.6) (layers F.Cu B.Cu) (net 7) (status 30))
 (segment (start 85.07 101.45) (end 80.01 101.45) (width 0.7) (layer B.Cu) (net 7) (status 10))
 (via (at 85.07 99.45) (size 1) (drill 0.6) (layers F.Cu B.Cu) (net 6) (status 30))
 (segment (start 69.87 99.45) (end 68.19 99.45) (width 0.5) (layer B.Cu) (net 3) (status 10))
 (segment (start 63.5 104.14) (end 59.69 104.14) (width 0.5) (layer B.Cu) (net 3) (status 20))
 (segment (start 68.19 99.45) (end 63.5 104.14) (width 0.5) (layer B.Cu) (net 3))
 (segment (start 72.54 101.45) (end 69.87 101.45) (width 0.5) (layer B.Cu) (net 2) (status 20))
 (segment (start 73.025 100.965) (end 72.54 101.45) (width 0.5) (layer B.Cu) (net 2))
 (via (at 73.025 100.965) (size 1) (drill 0.6) (layers F.Cu B.Cu) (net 2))
 (segment (start 75.13 95.685) (end 77.978 95.685) (width 0.5) (layer F.Cu) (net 2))
 (segment (start 73.66 97.155) (end 75.13 95.685) (width 0.5) (layer F.Cu) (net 2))
 (segment (start 77.978 95.685) (end 80.264 93.399) (width 0.5) (layer F.Cu) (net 2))
 (segment (start 73.66 100.33) (end 73.66 97.155) (width 0.5) (layer F.Cu) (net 2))
 (segment (start 73.025 100.965) (end 73.66 100.33) (width 0.5) (layer F.Cu) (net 2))
 (via (at 80.264 93.399) (size 1) (drill 0.6) (layers F.Cu B.Cu) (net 2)))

